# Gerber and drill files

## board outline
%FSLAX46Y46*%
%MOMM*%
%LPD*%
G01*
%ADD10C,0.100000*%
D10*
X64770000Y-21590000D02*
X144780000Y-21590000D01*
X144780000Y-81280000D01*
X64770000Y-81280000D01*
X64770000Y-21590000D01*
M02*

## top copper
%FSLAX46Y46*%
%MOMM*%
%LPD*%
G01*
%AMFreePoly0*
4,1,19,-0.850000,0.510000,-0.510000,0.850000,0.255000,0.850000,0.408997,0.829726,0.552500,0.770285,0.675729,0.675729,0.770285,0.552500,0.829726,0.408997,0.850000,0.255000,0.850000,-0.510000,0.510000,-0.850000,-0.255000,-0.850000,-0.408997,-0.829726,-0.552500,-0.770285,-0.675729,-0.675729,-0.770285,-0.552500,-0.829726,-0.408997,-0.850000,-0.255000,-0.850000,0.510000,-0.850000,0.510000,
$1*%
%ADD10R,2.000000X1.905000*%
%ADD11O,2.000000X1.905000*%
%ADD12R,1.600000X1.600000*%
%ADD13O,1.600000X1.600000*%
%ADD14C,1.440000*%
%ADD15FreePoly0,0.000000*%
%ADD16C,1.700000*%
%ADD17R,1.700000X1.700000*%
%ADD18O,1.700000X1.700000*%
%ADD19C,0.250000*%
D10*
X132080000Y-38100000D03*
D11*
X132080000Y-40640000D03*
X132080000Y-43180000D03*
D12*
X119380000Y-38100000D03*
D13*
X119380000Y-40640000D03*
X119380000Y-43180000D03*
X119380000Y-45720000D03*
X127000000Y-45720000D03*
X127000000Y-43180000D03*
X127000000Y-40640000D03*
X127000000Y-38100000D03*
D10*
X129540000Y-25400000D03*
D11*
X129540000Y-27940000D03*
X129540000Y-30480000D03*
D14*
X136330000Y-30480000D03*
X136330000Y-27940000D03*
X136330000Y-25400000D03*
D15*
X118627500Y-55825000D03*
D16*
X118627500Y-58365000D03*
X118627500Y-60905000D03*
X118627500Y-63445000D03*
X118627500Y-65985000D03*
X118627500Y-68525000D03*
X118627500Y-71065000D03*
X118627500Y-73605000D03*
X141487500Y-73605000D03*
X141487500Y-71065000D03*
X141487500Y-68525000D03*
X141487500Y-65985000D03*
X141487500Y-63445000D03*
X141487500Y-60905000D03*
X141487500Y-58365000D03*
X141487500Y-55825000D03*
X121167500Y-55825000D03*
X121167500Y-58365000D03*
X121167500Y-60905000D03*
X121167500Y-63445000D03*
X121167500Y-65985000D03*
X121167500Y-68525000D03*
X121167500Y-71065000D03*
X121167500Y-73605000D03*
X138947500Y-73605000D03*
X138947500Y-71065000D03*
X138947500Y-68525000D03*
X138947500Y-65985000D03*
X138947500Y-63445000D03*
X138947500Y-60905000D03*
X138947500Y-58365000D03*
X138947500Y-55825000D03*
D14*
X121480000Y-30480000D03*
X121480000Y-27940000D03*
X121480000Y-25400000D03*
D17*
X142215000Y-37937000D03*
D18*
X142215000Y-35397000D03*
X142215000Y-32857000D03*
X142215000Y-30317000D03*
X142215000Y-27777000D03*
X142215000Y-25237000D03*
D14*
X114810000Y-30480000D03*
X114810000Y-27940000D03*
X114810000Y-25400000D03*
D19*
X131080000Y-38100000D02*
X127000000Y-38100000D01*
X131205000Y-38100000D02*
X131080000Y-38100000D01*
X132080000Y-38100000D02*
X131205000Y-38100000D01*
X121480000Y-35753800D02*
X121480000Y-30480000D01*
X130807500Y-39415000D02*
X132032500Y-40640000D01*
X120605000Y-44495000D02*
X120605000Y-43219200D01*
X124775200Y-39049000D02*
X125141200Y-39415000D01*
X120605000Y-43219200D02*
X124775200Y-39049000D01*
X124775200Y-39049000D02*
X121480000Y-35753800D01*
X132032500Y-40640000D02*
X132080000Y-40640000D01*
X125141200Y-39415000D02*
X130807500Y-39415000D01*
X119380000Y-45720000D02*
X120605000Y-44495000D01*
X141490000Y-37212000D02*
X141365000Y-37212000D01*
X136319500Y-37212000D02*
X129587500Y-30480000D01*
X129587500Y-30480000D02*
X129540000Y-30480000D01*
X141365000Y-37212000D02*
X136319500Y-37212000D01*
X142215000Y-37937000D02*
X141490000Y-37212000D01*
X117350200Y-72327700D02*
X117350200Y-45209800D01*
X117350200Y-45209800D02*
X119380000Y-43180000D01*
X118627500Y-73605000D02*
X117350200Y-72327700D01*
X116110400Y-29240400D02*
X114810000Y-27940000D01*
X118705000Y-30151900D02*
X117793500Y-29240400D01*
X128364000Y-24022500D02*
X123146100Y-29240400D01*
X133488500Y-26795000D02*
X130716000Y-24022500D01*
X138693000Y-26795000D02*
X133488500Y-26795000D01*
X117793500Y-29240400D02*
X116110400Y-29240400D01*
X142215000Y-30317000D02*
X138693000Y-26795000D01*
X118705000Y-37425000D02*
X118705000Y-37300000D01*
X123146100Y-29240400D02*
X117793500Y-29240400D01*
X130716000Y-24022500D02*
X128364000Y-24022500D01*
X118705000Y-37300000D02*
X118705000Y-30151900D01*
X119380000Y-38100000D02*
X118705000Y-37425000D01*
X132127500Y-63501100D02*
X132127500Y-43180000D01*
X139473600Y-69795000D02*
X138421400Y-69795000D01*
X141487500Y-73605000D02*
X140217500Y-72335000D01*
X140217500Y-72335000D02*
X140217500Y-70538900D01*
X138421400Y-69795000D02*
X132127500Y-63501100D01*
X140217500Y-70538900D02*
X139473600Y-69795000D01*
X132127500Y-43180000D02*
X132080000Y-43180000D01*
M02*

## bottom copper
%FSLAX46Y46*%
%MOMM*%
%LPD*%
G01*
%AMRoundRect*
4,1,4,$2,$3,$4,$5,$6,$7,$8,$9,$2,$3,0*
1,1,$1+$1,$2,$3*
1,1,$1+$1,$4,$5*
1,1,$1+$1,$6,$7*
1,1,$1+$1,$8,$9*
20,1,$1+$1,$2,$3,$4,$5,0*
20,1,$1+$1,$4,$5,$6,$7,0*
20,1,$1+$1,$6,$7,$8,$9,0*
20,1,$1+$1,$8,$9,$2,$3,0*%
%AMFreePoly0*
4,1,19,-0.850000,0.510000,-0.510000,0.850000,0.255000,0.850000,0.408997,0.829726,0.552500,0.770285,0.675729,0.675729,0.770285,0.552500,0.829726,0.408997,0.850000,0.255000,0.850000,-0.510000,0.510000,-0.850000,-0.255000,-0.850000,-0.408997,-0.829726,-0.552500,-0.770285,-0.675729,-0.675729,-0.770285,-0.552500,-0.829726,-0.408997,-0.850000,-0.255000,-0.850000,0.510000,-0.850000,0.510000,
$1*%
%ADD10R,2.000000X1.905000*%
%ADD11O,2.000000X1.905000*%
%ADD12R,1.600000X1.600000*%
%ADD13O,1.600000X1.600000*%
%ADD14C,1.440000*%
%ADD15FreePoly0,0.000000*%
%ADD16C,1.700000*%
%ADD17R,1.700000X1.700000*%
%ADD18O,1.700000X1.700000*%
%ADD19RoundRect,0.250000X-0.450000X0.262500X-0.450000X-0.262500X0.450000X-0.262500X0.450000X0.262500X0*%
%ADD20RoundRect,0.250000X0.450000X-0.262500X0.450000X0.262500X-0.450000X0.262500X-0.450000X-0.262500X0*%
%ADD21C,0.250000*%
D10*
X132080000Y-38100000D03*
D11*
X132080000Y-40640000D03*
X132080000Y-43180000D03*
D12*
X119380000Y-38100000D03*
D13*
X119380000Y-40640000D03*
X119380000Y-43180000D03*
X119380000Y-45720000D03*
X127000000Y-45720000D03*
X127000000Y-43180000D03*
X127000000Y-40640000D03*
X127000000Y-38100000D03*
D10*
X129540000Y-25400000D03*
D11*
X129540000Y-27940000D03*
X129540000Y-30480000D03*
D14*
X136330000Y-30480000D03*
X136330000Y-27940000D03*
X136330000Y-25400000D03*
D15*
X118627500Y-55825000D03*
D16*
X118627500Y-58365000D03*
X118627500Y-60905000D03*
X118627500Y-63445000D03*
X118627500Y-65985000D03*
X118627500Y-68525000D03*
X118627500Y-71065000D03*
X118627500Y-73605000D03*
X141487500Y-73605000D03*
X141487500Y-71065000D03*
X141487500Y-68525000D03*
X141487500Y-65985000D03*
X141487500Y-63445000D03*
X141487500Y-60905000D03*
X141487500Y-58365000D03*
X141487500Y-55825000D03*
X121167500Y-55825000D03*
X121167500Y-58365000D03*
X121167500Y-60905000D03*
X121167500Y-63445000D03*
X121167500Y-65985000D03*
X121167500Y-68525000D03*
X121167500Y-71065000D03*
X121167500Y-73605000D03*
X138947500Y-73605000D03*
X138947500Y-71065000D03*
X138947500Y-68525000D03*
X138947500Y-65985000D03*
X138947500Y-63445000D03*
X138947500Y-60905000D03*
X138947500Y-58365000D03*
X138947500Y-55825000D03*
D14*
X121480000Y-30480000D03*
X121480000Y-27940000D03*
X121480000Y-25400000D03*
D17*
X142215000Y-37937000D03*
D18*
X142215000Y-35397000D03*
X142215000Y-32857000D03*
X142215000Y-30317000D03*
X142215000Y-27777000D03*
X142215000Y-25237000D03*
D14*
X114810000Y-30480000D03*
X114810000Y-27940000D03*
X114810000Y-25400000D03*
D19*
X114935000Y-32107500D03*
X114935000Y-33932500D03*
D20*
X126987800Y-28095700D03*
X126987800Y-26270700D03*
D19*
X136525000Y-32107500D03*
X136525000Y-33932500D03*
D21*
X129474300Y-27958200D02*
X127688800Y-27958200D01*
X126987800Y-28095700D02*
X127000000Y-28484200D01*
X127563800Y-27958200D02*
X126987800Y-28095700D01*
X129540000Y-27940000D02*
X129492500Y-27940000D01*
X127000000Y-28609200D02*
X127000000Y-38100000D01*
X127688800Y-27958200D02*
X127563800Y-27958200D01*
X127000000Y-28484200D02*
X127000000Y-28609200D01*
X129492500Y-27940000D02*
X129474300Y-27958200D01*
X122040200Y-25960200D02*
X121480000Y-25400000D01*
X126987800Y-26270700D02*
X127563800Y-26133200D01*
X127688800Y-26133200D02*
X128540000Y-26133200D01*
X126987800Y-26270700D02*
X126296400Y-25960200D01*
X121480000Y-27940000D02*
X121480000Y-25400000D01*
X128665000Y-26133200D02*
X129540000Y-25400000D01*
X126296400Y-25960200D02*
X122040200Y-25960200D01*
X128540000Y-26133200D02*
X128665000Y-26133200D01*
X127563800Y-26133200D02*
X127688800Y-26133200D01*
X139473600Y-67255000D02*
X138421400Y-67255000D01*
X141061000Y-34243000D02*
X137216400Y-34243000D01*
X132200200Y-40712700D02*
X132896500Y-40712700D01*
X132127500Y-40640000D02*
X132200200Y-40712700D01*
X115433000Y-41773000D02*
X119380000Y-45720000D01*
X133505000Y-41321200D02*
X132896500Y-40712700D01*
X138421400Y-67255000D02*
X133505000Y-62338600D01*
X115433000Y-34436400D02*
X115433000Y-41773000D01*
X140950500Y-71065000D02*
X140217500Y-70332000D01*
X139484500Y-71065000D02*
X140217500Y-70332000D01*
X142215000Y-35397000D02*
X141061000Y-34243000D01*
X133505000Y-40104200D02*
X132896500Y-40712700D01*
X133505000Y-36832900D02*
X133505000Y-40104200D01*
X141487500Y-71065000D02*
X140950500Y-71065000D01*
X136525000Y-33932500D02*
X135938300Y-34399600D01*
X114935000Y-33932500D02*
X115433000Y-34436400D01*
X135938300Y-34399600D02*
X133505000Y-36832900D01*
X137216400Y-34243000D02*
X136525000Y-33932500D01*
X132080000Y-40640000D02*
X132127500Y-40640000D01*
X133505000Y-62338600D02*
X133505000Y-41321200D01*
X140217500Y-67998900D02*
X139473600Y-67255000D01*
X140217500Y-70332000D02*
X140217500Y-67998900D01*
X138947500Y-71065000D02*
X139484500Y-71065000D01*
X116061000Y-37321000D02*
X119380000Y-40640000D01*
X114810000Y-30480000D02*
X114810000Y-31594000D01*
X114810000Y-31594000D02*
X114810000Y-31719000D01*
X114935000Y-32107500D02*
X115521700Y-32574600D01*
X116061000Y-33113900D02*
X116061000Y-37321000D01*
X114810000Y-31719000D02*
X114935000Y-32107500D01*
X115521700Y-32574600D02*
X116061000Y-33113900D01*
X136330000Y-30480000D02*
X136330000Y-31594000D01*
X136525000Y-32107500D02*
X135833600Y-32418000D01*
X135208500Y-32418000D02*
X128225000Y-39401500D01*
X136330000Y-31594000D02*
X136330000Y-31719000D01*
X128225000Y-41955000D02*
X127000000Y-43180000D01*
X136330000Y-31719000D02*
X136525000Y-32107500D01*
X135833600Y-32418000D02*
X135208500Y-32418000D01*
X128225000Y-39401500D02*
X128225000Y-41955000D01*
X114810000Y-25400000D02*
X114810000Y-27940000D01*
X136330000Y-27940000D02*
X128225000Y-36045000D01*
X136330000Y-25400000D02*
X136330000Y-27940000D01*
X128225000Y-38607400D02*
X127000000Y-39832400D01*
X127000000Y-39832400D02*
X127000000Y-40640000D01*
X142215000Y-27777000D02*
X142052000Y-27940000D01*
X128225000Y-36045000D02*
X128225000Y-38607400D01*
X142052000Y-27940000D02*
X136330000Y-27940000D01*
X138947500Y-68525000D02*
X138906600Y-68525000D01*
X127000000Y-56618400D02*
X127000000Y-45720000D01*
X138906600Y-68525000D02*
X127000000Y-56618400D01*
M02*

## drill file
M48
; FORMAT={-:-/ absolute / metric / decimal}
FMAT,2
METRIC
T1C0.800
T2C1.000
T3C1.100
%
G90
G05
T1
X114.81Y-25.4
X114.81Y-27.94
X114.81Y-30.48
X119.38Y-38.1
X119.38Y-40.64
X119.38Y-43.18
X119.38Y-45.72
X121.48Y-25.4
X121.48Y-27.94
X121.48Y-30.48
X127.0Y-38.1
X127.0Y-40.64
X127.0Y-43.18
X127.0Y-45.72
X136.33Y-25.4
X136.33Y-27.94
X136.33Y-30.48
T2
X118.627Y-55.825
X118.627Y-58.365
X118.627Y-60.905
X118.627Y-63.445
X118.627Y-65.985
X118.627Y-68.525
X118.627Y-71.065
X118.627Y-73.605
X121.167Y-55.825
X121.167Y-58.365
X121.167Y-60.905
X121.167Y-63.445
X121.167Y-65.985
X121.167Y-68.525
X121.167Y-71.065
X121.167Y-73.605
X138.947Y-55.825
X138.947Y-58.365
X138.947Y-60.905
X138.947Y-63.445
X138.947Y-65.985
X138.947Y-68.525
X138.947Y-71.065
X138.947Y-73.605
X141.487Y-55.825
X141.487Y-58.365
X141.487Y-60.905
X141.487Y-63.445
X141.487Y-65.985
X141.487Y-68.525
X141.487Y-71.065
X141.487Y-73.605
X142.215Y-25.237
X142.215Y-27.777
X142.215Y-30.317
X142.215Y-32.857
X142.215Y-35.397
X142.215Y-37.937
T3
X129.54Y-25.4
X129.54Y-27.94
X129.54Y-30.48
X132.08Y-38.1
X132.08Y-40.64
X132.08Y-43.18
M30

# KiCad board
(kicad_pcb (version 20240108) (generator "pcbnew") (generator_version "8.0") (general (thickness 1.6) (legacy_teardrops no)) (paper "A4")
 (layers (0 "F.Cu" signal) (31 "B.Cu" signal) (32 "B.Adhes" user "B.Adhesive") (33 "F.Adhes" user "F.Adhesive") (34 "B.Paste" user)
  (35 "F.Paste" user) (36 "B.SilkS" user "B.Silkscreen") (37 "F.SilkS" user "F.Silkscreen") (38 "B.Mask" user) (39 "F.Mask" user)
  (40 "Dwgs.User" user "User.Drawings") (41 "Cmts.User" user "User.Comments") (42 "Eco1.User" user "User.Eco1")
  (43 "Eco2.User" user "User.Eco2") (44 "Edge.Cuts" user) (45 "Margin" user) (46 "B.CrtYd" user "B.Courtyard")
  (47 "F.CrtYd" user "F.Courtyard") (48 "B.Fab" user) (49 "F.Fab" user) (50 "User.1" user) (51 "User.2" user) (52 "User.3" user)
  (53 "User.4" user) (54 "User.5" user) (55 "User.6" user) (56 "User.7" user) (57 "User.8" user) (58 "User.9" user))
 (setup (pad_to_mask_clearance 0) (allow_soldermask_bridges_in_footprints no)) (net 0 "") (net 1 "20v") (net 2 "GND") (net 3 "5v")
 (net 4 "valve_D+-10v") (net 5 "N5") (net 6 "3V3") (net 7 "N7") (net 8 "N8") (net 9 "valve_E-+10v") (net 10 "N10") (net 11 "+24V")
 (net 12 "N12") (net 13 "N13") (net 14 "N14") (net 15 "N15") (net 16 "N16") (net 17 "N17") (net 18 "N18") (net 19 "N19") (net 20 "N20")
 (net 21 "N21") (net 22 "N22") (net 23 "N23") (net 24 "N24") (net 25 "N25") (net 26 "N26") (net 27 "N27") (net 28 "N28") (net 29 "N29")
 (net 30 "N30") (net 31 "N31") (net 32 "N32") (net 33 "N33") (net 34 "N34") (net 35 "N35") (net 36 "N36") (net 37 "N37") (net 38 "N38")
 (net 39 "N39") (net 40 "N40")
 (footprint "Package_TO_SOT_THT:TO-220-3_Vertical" (layer "F.Cu") (at 132.08 38.1 -90)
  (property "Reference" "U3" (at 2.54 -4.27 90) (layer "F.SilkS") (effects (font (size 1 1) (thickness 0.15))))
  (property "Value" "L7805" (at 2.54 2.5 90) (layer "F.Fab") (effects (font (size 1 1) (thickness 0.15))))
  (pad "1" thru_hole rect (at 0 0 270) (size 1.905 2) (drill 1.1) (layers "*.Cu" "*.Mask") (remove_unused_layers no) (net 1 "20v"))
  (pad "2" thru_hole oval (at 2.54 0 270) (size 1.905 2) (drill 1.1) (layers "*.Cu" "*.Mask") (remove_unused_layers no) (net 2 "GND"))
  (pad "3" thru_hole oval (at 5.08 0 270) (size 1.905 2) (drill 1.1) (layers "*.Cu" "*.Mask") (remove_unused_layers no) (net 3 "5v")))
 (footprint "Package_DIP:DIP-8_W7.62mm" (layer "F.Cu") (at 119.38 38.1)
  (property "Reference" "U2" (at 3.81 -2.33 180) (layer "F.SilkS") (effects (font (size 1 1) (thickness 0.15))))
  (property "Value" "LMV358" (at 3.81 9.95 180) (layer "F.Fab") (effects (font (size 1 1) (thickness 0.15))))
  (pad "1" thru_hole rect (at 0 0) (size 1.6 1.6) (drill 0.8) (layers "*.Cu" "*.Mask") (remove_unused_layers no) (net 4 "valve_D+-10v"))
  (pad "2" thru_hole oval (at 0 2.54) (size 1.6 1.6) (drill 0.8) (layers "*.Cu" "*.Mask") (remove_unused_layers no) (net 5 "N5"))
  (pad "3" thru_hole oval (at 0 5.08) (size 1.6 1.6) (drill 0.8) (layers "*.Cu" "*.Mask") (remove_unused_layers no) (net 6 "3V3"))
  (pad "4" thru_hole oval (at 0 7.62) (size 1.6 1.6) (drill 0.8) (layers "*.Cu" "*.Mask") (remove_unused_layers no) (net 2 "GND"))
  (pad "5" thru_hole oval (at 7.62 7.62) (size 1.6 1.6) (drill 0.8) (layers "*.Cu" "*.Mask") (remove_unused_layers no) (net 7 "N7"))
  (pad "6" thru_hole oval (at 7.62 5.08) (size 1.6 1.6) (drill 0.8) (layers "*.Cu" "*.Mask") (remove_unused_layers no) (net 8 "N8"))
  (pad "7" thru_hole oval (at 7.62 2.54) (size 1.6 1.6) (drill 0.8) (layers "*.Cu" "*.Mask") (remove_unused_layers no)
   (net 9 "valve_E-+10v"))
  (pad "8" thru_hole oval (at 7.62 0) (size 1.6 1.6) (drill 0.8) (layers "*.Cu" "*.Mask") (remove_unused_layers no) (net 1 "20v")))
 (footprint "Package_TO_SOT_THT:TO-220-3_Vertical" (layer "F.Cu") (at 129.54 25.4 -90)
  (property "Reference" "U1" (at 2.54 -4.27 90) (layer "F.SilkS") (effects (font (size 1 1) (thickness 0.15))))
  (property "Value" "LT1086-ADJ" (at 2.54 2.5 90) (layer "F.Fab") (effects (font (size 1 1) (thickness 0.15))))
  (pad "1" thru_hole rect (at 0 0 270) (size 1.905 2) (drill 1.1) (layers "*.Cu" "*.Mask") (remove_unused_layers no) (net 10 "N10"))
  (pad "2" thru_hole oval (at 2.54 0 270) (size 1.905 2) (drill 1.1) (layers "*.Cu" "*.Mask") (remove_unused_layers no) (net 1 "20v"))
  (pad "3" thru_hole oval (at 5.08 0 270) (size 1.905 2) (drill 1.1) (layers "*.Cu" "*.Mask") (remove_unused_layers no) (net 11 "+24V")))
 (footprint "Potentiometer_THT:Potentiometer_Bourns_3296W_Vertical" (layer "F.Cu") (at 136.33 30.48 -90)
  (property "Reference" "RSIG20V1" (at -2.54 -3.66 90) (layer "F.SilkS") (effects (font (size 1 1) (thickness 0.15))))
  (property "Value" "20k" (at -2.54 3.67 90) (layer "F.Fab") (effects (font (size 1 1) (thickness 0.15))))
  (pad "1" thru_hole circle (at 0 0 270) (size 1.44 1.44) (drill 0.8) (layers "*.Cu" "*.Mask") (remove_unused_layers no) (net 8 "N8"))
  (pad "2" thru_hole circle (at -2.54 0 270) (size 1.44 1.44) (drill 0.8) (layers "*.Cu" "*.Mask") (remove_unused_layers no)
   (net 9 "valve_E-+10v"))
  (pad "3" thru_hole circle (at -5.08 0 270) (size 1.44 1.44) (drill 0.8) (layers "*.Cu" "*.Mask") (remove_unused_layers no)
   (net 9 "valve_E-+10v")))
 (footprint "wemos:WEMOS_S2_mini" (layer "F.Cu") (at 118.6275 55.825)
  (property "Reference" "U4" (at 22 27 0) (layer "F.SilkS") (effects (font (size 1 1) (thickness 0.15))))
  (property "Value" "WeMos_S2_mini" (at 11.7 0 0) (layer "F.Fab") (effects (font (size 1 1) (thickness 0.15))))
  (pad "1" thru_hole roundrect (at 0 0) (size 1.7 1.7) (drill 1) (layers "*.Cu" "*.Mask") (remove_unused_layers no) (roundrect_rratio 0.35)
   (chamfer_ratio 0.2) (chamfer top_left bottom_right) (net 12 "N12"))
  (pad "2" thru_hole circle (at 0 2.54) (size 1.7 1.7) (drill 1) (layers "*.Cu" "*.Mask") (remove_unused_layers no) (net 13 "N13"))
  (pad "3" thru_hole circle (at 0 5.08) (size 1.7 1.7) (drill 1) (layers "*.Cu" "*.Mask") (remove_unused_layers no) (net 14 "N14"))
  (pad "4" thru_hole circle (at 0 7.62) (size 1.7 1.7) (drill 1) (layers "*.Cu" "*.Mask") (remove_unused_layers no) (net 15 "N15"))
  (pad "5" thru_hole circle (at 0 10.16) (size 1.7 1.7) (drill 1) (layers "*.Cu" "*.Mask") (remove_unused_layers no) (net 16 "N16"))
  (pad "6" thru_hole circle (at 0 12.7) (size 1.7 1.7) (drill 1) (layers "*.Cu" "*.Mask") (remove_unused_layers no) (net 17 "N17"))
  (pad "7" thru_hole circle (at 0 15.24) (size 1.7 1.7) (drill 1) (layers "*.Cu" "*.Mask") (remove_unused_layers no) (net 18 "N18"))
  (pad "8" thru_hole circle (at 0 17.78) (size 1.7 1.7) (drill 1) (layers "*.Cu" "*.Mask") (remove_unused_layers no) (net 6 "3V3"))
  (pad "9" thru_hole circle (at 22.86 17.78) (size 1.7 1.7) (drill 1) (layers "*.Cu" "*.Mask") (remove_unused_layers no) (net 3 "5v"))
  (pad "10" thru_hole circle (at 22.86 15.24) (size 1.7 1.7) (drill 1) (layers "*.Cu" "*.Mask") (remove_unused_layers no) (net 2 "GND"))
  (pad "11" thru_hole circle (at 22.86 12.7) (size 1.7 1.7) (drill 1) (layers "*.Cu" "*.Mask") (remove_unused_layers no) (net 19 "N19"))
  (pad "12" thru_hole circle (at 22.86 10.16) (size 1.7 1.7) (drill 1) (layers "*.Cu" "*.Mask") (remove_unused_layers no) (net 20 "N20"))
  (pad "13" thru_hole circle (at 22.86 7.62) (size 1.7 1.7) (drill 1) (layers "*.Cu" "*.Mask") (remove_unused_layers no) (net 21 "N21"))
  (pad "14" thru_hole circle (at 22.86 5.08) (size 1.7 1.7) (drill 1) (layers "*.Cu" "*.Mask") (remove_unused_layers no) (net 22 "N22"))
  (pad "15" thru_hole circle (at 22.86 2.54) (size 1.7 1.7) (drill 1) (layers "*.Cu" "*.Mask") (remove_unused_layers no) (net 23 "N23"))
  (pad "16" thru_hole circle (at 22.86 0) (size 1.7 1.7) (drill 1) (layers "*.Cu" "*.Mask") (remove_unused_layers no) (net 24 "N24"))
  (pad "17" thru_hole circle (at 2.54 0) (size 1.7 1.7) (drill 1) (layers "*.Cu" "*.Mask") (remove_unused_layers no) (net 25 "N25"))
  (pad "18" thru_hole circle (at 2.54 2.54) (size 1.7 1.7) (drill 1) (layers "*.Cu" "*.Mask") (remove_unused_layers no) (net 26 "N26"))
  (pad "19" thru_hole circle (at 2.54 5.08) (size 1.7 1.7) (drill 1) (layers "*.Cu" "*.Mask") (remove_unused_layers no) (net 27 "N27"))
  (pad "20" thru_hole circle (at 2.54 7.62) (size 1.7 1.7) (drill 1) (layers "*.Cu" "*.Mask") (remove_unused_layers no) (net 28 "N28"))
  (pad "21" thru_hole circle (at 2.54 10.16) (size 1.7 1.7) (drill 1) (layers "*.Cu" "*.Mask") (remove_unused_layers no) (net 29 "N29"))
  (pad "22" thru_hole circle (at 2.54 12.7) (size 1.7 1.7) (drill 1) (layers "*.Cu" "*.Mask") (remove_unused_layers no) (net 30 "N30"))
  (pad "23" thru_hole circle (at 2.54 15.24) (size 1.7 1.7) (drill 1) (layers "*.Cu" "*.Mask") (remove_unused_layers no) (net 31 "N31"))
  (pad "24" thru_hole circle (at 2.54 17.78) (size 1.7 1.7) (drill 1) (layers "*.Cu" "*.Mask") (remove_unused_layers no) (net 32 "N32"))
  (pad "25" thru_hole circle (at 20.32 17.78) (size 1.7 1.7) (drill 1) (layers "*.Cu" "*.Mask") (remove_unused_layers no) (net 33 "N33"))
  (pad "26" thru_hole circle (at 20.32 15.24) (size 1.7 1.7) (drill 1) (layers "*.Cu" "*.Mask") (remove_unused_layers no) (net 2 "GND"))
  (pad "27" thru_hole circle (at 20.32 12.7) (size 1.7 1.7) (drill 1) (layers "*.Cu" "*.Mask") (remove_unused_layers no) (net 7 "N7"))
  (pad "28" thru_hole circle (at 20.32 10.16) (size 1.7 1.7) (drill 1) (layers "*.Cu" "*.Mask") (remove_unused_layers no) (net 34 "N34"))
  (pad "29" thru_hole circle (at 20.32 7.62) (size 1.7 1.7) (drill 1) (layers "*.Cu" "*.Mask") (remove_unused_layers no) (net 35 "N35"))
  (pad "30" thru_hole circle (at 20.32 5.08) (size 1.7 1.7) (drill 1) (layers "*.Cu" "*.Mask") (remove_unused_layers no) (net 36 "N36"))
  (pad "31" thru_hole circle (at 20.32 2.54) (size 1.7 1.7) (drill 1) (layers "*.Cu" "*.Mask") (remove_unused_layers no) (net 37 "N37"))
  (pad "32" thru_hole circle (at 20.32 0) (size 1.7 1.7) (drill 1) (layers "*.Cu" "*.Mask") (remove_unused_layers no) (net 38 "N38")))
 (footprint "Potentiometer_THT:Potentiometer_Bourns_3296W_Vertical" (layer "F.Cu") (at 121.48 30.48 -90)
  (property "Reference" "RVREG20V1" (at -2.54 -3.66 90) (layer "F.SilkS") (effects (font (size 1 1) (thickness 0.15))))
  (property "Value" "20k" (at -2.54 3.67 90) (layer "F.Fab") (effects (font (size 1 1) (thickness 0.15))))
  (pad "1" thru_hole circle (at 0 0 270) (size 1.44 1.44) (drill 0.8) (layers "*.Cu" "*.Mask") (remove_unused_layers no) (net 2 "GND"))
  (pad "2" thru_hole circle (at -2.54 0 270) (size 1.44 1.44) (drill 0.8) (layers "*.Cu" "*.Mask") (remove_unused_layers no) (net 10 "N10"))
  (pad "3" thru_hole circle (at -5.08 0 270) (size 1.44 1.44) (drill 0.8) (layers "*.Cu" "*.Mask") (remove_unused_layers no) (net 10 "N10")))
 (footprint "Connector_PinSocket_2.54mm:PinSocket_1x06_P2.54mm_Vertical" (layer "F.Cu") (at 142.215 37.937 180)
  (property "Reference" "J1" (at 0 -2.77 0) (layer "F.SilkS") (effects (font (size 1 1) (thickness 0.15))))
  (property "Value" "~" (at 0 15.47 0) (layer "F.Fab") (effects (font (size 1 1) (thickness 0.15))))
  (pad "1" thru_hole rect (at 0 0 180) (size 1.7 1.7) (drill 1) (layers "*.Cu" "*.Mask") (remove_unused_layers no) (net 11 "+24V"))
  (pad "2" thru_hole oval (at 0 2.54 180) (size 1.7 1.7) (drill 1) (layers "*.Cu" "*.Mask") (remove_unused_layers no) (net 2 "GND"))
  (pad "3" thru_hole oval (at 0 5.08 180) (size 1.7 1.7) (drill 1) (layers "*.Cu" "*.Mask") (remove_unused_layers no) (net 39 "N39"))
  (pad "4" thru_hole oval (at 0 7.62 180) (size 1.7 1.7) (drill 1) (layers "*.Cu" "*.Mask") (remove_unused_layers no) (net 4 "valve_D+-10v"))
  (pad "5" thru_hole oval (at 0 10.16 180) (size 1.7 1.7) (drill 1) (layers "*.Cu" "*.Mask") (remove_unused_layers no)
   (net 9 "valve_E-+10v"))
  (pad "6" thru_hole oval (at 0 12.7 180) (size 1.7 1.7) (drill 1) (layers "*.Cu" "*.Mask") (remove_unused_layers no) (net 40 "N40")))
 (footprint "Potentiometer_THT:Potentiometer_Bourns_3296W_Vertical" (layer "F.Cu") (at 114.81 30.48 -90)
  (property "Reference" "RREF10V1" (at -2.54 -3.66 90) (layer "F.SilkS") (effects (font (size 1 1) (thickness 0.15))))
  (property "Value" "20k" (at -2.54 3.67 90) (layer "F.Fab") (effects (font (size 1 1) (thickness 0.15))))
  (pad "1" thru_hole circle (at 0 0 270) (size 1.44 1.44) (drill 0.8) (layers "*.Cu" "*.Mask") (remove_unused_layers no) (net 5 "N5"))
  (pad "2" thru_hole circle (at -2.54 0 270) (size 1.44 1.44) (drill 0.8) (layers "*.Cu" "*.Mask") (remove_unused_layers no)
   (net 4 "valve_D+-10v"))
  (pad "3" thru_hole circle (at -5.08 0 270) (size 1.44 1.44) (drill 0.8) (layers "*.Cu" "*.Mask") (remove_unused_layers no)
   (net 4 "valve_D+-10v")))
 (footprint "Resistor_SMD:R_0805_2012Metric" (layer "B.Cu") (at 114.935 33.02 -90)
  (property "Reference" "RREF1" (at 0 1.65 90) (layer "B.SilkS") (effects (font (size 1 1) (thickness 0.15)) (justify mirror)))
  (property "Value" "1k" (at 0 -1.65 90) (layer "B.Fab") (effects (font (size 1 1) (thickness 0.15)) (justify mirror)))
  (pad "1" smd roundrect (at -0.9125 0 270) (size 1.025 1.4) (layers "B.Cu" "B.Paste" "B.Mask") (roundrect_rratio 0.243902) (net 5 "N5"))
  (pad "2" smd roundrect (at 0.9125 0 270) (size 1.025 1.4) (layers "B.Cu" "B.Paste" "B.Mask") (roundrect_rratio 0.243902) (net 2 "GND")))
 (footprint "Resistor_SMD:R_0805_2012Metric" (layer "B.Cu") (at 126.9878 27.1832 90)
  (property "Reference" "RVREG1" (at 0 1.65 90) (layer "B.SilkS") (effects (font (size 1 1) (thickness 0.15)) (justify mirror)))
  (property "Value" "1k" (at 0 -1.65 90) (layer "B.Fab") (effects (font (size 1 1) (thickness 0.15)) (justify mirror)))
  (pad "1" smd roundrect (at -0.9125 0 90) (size 1.025 1.4) (layers "B.Cu" "B.Paste" "B.Mask") (roundrect_rratio 0.243902) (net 1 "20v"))
  (pad "2" smd roundrect (at 0.9125 0 90) (size 1.025 1.4) (layers "B.Cu" "B.Paste" "B.Mask") (roundrect_rratio 0.243902) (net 10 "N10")))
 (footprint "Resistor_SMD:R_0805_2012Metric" (layer "B.Cu") (at 136.525 33.02 -90)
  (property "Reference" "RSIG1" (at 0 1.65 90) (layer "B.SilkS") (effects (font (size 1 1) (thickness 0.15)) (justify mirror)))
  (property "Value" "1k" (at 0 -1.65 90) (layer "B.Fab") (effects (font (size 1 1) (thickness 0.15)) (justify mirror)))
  (pad "1" smd roundrect (at -0.9125 0 270) (size 1.025 1.4) (layers "B.Cu" "B.Paste" "B.Mask") (roundrect_rratio 0.243902) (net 8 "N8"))
  (pad "2" smd roundrect (at 0.9125 0 270) (size 1.025 1.4) (layers "B.Cu" "B.Paste" "B.Mask") (roundrect_rratio 0.243902) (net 2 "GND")))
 (gr_rect (start 64.77 21.59) (end 144.78 81.28) (stroke (width 0.1) (type default)) (fill none) (layer "Edge.Cuts"))
 (segment (start 131.08 38.1) (end 127 38.1) (width 0.25) (layer "F.Cu") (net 1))
 (segment (start 131.205 38.1) (end 131.08 38.1) (width 0.25) (layer "F.Cu") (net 1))
 (segment (start 132.08 38.1) (end 131.205 38.1) (width 0.25) (layer "F.Cu") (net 1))
 (segment (start 129.4743 27.9582) (end 127.6888 27.9582) (width 0.25) (layer "B.Cu") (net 1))
 (segment (start 126.9878 28.0957) (end 127 28.4842) (width 0.25) (layer "B.Cu") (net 1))
 (segment (start 127.5638 27.9582) (end 126.9878 28.0957) (width 0.25) (layer "B.Cu") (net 1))
 (segment (start 129.54 27.94) (end 129.4925 27.94) (width 0.25) (layer "B.Cu") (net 1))
 (segment (start 127 28.6092) (end 127 38.1) (width 0.25) (layer "B.Cu") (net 1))
 (segment (start 127.6888 27.9582) (end 127.5638 27.9582) (width 0.25) (layer "B.Cu") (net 1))
 (segment (start 127 28.4842) (end 127 28.6092) (width 0.25) (layer "B.Cu") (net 1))
 (segment (start 129.4925 27.94) (end 129.4743 27.9582) (width 0.25) (layer "B.Cu") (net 1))
 (segment (start 122.0402 25.9602) (end 121.48 25.4) (width 0.25) (layer "B.Cu") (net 10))
 (segment (start 126.9878 26.2707) (end 127.5638 26.1332) (width 0.25) (layer "B.Cu") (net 10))
 (segment (start 127.6888 26.1332) (end 128.54 26.1332) (width 0.25) (layer "B.Cu") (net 10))
 (segment (start 126.9878 26.2707) (end 126.2964 25.9602) (width 0.25) (layer "B.Cu") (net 10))
 (segment (start 121.48 27.94) (end 121.48 25.4) (width 0.25) (layer "B.Cu") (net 10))
 (segment (start 128.665 26.1332) (end 129.54 25.4) (width 0.25) (layer "B.Cu") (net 10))
 (segment (start 126.2964 25.9602) (end 122.0402 25.9602) (width 0.25) (layer "B.Cu") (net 10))
 (segment (start 128.54 26.1332) (end 128.665 26.1332) (width 0.25) (layer "B.Cu") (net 10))
 (segment (start 127.5638 26.1332) (end 127.6888 26.1332) (width 0.25) (layer "B.Cu") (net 10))
 (segment (start 121.48 35.7538) (end 121.48 30.48) (width 0.25) (layer "F.Cu") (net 2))
 (segment (start 130.8075 39.415) (end 132.0325 40.64) (width 0.25) (layer "F.Cu") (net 2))
 (segment (start 120.605 44.495) (end 120.605 43.2192) (width 0.25) (layer "F.Cu") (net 2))
 (segment (start 124.7752 39.049) (end 125.1412 39.415) (width 0.25) (layer "F.Cu") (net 2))
 (segment (start 120.605 43.2192) (end 124.7752 39.049) (width 0.25) (layer "F.Cu") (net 2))
 (segment (start 124.7752 39.049) (end 121.48 35.7538) (width 0.25) (layer "F.Cu") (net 2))
 (segment (start 132.0325 40.64) (end 132.08 40.64) (width 0.25) (layer "F.Cu") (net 2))
 (segment (start 125.1412 39.415) (end 130.8075 39.415) (width 0.25) (layer "F.Cu") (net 2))
 (segment (start 119.38 45.72) (end 120.605 44.495) (width 0.25) (layer "F.Cu") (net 2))
 (segment (start 139.4736 67.255) (end 138.4214 67.255) (width 0.25) (layer "B.Cu") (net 2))
 (segment (start 141.061 34.243) (end 137.2164 34.243) (width 0.25) (layer "B.Cu") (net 2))
 (segment (start 132.2002 40.7127) (end 132.8965 40.7127) (width 0.25) (layer "B.Cu") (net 2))
 (segment (start 132.1275 40.64) (end 132.2002 40.7127) (width 0.25) (layer "B.Cu") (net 2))
 (segment (start 115.433 41.773) (end 119.38 45.72) (width 0.25) (layer "B.Cu") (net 2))
 (segment (start 133.505 41.3212) (end 132.8965 40.7127) (width 0.25) (layer "B.Cu") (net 2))
 (segment (start 138.4214 67.255) (end 133.505 62.3386) (width 0.25) (layer "B.Cu") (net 2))
 (segment (start 115.433 34.4364) (end 115.433 41.773) (width 0.25) (layer "B.Cu") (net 2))
 (segment (start 140.9505 71.065) (end 140.2175 70.332) (width 0.25) (layer "B.Cu") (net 2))
 (segment (start 139.4845 71.065) (end 140.2175 70.332) (width 0.25) (layer "B.Cu") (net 2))
 (segment (start 142.215 35.397) (end 141.061 34.243) (width 0.25) (layer "B.Cu") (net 2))
 (segment (start 133.505 40.1042) (end 132.8965 40.7127) (width 0.25) (layer "B.Cu") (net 2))
 (segment (start 133.505 36.8329) (end 133.505 40.1042) (width 0.25) (layer "B.Cu") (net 2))
 (segment (start 141.4875 71.065) (end 140.9505 71.065) (width 0.25) (layer "B.Cu") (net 2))
 (segment (start 136.525 33.9325) (end 135.9383 34.3996) (width 0.25) (layer "B.Cu") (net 2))
 (segment (start 114.935 33.9325) (end 115.433 34.4364) (width 0.25) (layer "B.Cu") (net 2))
 (segment (start 135.9383 34.3996) (end 133.505 36.8329) (width 0.25) (layer "B.Cu") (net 2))
 (segment (start 137.2164 34.243) (end 136.525 33.9325) (width 0.25) (layer "B.Cu") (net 2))
 (segment (start 132.08 40.64) (end 132.1275 40.64) (width 0.25) (layer "B.Cu") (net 2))
 (segment (start 133.505 62.3386) (end 133.505 41.3212) (width 0.25) (layer "B.Cu") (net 2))
 (segment (start 140.2175 67.9989) (end 139.4736 67.255) (width 0.25) (layer "B.Cu") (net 2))
 (segment (start 140.2175 70.332) (end 140.2175 67.9989) (width 0.25) (layer "B.Cu") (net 2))
 (segment (start 138.9475 71.065) (end 139.4845 71.065) (width 0.25) (layer "B.Cu") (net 2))
 (segment (start 141.49 37.212) (end 141.365 37.212) (width 0.25) (layer "F.Cu") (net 11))
 (segment (start 136.3195 37.212) (end 129.5875 30.48) (width 0.25) (layer "F.Cu") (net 11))
 (segment (start 129.5875 30.48) (end 129.54 30.48) (width 0.25) (layer "F.Cu") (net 11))
 (segment (start 141.365 37.212) (end 136.3195 37.212) (width 0.25) (layer "F.Cu") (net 11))
 (segment (start 142.215 37.937) (end 141.49 37.212) (width 0.25) (layer "F.Cu") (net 11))
 (segment (start 116.061 37.321) (end 119.38 40.64) (width 0.25) (layer "B.Cu") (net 5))
 (segment (start 114.81 30.48) (end 114.81 31.594) (width 0.25) (layer "B.Cu") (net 5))
 (segment (start 114.81 31.594) (end 114.81 31.719) (width 0.25) (layer "B.Cu") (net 5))
 (segment (start 114.935 32.1075) (end 115.5217 32.5746) (width 0.25) (layer "B.Cu") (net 5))
 (segment (start 116.061 33.1139) (end 116.061 37.321) (width 0.25) (layer "B.Cu") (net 5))
 (segment (start 114.81 31.719) (end 114.935 32.1075) (width 0.25) (layer "B.Cu") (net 5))
 (segment (start 115.5217 32.5746) (end 116.061 33.1139) (width 0.25) (layer "B.Cu") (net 5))
 (segment (start 117.3502 72.3277) (end 117.3502 45.2098) (width 0.25) (layer "F.Cu") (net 6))
 (segment (start 117.3502 45.2098) (end 119.38 43.18) (width 0.25) (layer "F.Cu") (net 6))
 (segment (start 118.6275 73.605) (end 117.3502 72.3277) (width 0.25) (layer "F.Cu") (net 6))
 (segment (start 136.33 30.48) (end 136.33 31.594) (width 0.25) (layer "B.Cu") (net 8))
 (segment (start 136.525 32.1075) (end 135.8336 32.418) (width 0.25) (layer "B.Cu") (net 8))
 (segment (start 135.2085 32.418) (end 128.225 39.4015) (width 0.25) (layer "B.Cu") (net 8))
 (segment (start 136.33 31.594) (end 136.33 31.719) (width 0.25) (layer "B.Cu") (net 8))
 (segment (start 128.225 41.955) (end 127 43.18) (width 0.25) (layer "B.Cu") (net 8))
 (segment (start 136.33 31.719) (end 136.525 32.1075) (width 0.25) (layer "B.Cu") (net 8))
 (segment (start 135.8336 32.418) (end 135.2085 32.418) (width 0.25) (layer "B.Cu") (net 8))
 (segment (start 128.225 39.4015) (end 128.225 41.955) (width 0.25) (layer "B.Cu") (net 8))
 (segment (start 116.1104 29.2404) (end 114.81 27.94) (width 0.25) (layer "F.Cu") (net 4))
 (segment (start 118.705 30.1519) (end 117.7935 29.2404) (width 0.25) (layer "F.Cu") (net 4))
 (segment (start 128.364 24.0225) (end 123.1461 29.2404) (width 0.25) (layer "F.Cu") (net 4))
 (segment (start 133.4885 26.795) (end 130.716 24.0225) (width 0.25) (layer "F.Cu") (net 4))
 (segment (start 138.693 26.795) (end 133.4885 26.795) (width 0.25) (layer "F.Cu") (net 4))
 (segment (start 117.7935 29.2404) (end 116.1104 29.2404) (width 0.25) (layer "F.Cu") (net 4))
 (segment (start 142.215 30.317) (end 138.693 26.795) (width 0.25) (layer "F.Cu") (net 4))
 (segment (start 118.705 37.425) (end 118.705 37.3) (width 0.25) (layer "F.Cu") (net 4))
 (segment (start 123.1461 29.2404) (end 117.7935 29.2404) (width 0.25) (layer "F.Cu") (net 4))
 (segment (start 130.716 24.0225) (end 128.364 24.0225) (width 0.25) (layer "F.Cu") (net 4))
 (segment (start 118.705 37.3) (end 118.705 30.1519) (width 0.25) (layer "F.Cu") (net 4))
 (segment (start 119.38 38.1) (end 118.705 37.425) (width 0.25) (layer "F.Cu") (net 4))
 (segment (start 114.81 25.4) (end 114.81 27.94) (width 0.25) (layer "B.Cu") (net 4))
 (segment (start 136.33 27.94) (end 128.225 36.045) (width 0.25) (layer "B.Cu") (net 9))
 (segment (start 136.33 25.4) (end 136.33 27.94) (width 0.25) (layer "B.Cu") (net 9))
 (segment (start 128.225 38.6074) (end 127 39.8324) (width 0.25) (layer "B.Cu") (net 9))
 (segment (start 127 39.8324) (end 127 40.64) (width 0.25) (layer "B.Cu") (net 9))
 (segment (start 142.215 27.777) (end 142.052 27.94) (width 0.25) (layer "B.Cu") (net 9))
 (segment (start 128.225 36.045) (end 128.225 38.6074) (width 0.25) (layer "B.Cu") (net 9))
 (segment (start 142.052 27.94) (end 136.33 27.94) (width 0.25) (layer "B.Cu") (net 9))
 (segment (start 132.1275 63.5011) (end 132.1275 43.18) (width 0.25) (layer "F.Cu") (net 3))
 (segment (start 139.4736 69.795) (end 138.4214 69.795) (width 0.25) (layer "F.Cu") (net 3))
 (segment (start 141.4875 73.605) (end 140.2175 72.335) (width 0.25) (layer "F.Cu") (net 3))
 (segment (start 140.2175 72.335) (end 140.2175 70.5389) (width 0.25) (layer "F.Cu") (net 3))
 (segment (start 138.4214 69.795) (end 132.1275 63.5011) (width 0.25) (layer "F.Cu") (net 3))
 (segment (start 140.2175 70.5389) (end 139.4736 69.795) (width 0.25) (layer "F.Cu") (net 3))
 (segment (start 132.1275 43.18) (end 132.08 43.18) (width 0.25) (layer "F.Cu") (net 3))
 (segment (start 138.9475 68.525) (end 138.9066 68.525) (width 0.25) (layer "B.Cu") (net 7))
 (segment (start 127 56.6184) (end 127 45.72) (width 0.25) (layer "B.Cu") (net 7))
 (segment (start 138.9066 68.525) (end 127 56.6184) (width 0.25) (layer "B.Cu") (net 7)))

